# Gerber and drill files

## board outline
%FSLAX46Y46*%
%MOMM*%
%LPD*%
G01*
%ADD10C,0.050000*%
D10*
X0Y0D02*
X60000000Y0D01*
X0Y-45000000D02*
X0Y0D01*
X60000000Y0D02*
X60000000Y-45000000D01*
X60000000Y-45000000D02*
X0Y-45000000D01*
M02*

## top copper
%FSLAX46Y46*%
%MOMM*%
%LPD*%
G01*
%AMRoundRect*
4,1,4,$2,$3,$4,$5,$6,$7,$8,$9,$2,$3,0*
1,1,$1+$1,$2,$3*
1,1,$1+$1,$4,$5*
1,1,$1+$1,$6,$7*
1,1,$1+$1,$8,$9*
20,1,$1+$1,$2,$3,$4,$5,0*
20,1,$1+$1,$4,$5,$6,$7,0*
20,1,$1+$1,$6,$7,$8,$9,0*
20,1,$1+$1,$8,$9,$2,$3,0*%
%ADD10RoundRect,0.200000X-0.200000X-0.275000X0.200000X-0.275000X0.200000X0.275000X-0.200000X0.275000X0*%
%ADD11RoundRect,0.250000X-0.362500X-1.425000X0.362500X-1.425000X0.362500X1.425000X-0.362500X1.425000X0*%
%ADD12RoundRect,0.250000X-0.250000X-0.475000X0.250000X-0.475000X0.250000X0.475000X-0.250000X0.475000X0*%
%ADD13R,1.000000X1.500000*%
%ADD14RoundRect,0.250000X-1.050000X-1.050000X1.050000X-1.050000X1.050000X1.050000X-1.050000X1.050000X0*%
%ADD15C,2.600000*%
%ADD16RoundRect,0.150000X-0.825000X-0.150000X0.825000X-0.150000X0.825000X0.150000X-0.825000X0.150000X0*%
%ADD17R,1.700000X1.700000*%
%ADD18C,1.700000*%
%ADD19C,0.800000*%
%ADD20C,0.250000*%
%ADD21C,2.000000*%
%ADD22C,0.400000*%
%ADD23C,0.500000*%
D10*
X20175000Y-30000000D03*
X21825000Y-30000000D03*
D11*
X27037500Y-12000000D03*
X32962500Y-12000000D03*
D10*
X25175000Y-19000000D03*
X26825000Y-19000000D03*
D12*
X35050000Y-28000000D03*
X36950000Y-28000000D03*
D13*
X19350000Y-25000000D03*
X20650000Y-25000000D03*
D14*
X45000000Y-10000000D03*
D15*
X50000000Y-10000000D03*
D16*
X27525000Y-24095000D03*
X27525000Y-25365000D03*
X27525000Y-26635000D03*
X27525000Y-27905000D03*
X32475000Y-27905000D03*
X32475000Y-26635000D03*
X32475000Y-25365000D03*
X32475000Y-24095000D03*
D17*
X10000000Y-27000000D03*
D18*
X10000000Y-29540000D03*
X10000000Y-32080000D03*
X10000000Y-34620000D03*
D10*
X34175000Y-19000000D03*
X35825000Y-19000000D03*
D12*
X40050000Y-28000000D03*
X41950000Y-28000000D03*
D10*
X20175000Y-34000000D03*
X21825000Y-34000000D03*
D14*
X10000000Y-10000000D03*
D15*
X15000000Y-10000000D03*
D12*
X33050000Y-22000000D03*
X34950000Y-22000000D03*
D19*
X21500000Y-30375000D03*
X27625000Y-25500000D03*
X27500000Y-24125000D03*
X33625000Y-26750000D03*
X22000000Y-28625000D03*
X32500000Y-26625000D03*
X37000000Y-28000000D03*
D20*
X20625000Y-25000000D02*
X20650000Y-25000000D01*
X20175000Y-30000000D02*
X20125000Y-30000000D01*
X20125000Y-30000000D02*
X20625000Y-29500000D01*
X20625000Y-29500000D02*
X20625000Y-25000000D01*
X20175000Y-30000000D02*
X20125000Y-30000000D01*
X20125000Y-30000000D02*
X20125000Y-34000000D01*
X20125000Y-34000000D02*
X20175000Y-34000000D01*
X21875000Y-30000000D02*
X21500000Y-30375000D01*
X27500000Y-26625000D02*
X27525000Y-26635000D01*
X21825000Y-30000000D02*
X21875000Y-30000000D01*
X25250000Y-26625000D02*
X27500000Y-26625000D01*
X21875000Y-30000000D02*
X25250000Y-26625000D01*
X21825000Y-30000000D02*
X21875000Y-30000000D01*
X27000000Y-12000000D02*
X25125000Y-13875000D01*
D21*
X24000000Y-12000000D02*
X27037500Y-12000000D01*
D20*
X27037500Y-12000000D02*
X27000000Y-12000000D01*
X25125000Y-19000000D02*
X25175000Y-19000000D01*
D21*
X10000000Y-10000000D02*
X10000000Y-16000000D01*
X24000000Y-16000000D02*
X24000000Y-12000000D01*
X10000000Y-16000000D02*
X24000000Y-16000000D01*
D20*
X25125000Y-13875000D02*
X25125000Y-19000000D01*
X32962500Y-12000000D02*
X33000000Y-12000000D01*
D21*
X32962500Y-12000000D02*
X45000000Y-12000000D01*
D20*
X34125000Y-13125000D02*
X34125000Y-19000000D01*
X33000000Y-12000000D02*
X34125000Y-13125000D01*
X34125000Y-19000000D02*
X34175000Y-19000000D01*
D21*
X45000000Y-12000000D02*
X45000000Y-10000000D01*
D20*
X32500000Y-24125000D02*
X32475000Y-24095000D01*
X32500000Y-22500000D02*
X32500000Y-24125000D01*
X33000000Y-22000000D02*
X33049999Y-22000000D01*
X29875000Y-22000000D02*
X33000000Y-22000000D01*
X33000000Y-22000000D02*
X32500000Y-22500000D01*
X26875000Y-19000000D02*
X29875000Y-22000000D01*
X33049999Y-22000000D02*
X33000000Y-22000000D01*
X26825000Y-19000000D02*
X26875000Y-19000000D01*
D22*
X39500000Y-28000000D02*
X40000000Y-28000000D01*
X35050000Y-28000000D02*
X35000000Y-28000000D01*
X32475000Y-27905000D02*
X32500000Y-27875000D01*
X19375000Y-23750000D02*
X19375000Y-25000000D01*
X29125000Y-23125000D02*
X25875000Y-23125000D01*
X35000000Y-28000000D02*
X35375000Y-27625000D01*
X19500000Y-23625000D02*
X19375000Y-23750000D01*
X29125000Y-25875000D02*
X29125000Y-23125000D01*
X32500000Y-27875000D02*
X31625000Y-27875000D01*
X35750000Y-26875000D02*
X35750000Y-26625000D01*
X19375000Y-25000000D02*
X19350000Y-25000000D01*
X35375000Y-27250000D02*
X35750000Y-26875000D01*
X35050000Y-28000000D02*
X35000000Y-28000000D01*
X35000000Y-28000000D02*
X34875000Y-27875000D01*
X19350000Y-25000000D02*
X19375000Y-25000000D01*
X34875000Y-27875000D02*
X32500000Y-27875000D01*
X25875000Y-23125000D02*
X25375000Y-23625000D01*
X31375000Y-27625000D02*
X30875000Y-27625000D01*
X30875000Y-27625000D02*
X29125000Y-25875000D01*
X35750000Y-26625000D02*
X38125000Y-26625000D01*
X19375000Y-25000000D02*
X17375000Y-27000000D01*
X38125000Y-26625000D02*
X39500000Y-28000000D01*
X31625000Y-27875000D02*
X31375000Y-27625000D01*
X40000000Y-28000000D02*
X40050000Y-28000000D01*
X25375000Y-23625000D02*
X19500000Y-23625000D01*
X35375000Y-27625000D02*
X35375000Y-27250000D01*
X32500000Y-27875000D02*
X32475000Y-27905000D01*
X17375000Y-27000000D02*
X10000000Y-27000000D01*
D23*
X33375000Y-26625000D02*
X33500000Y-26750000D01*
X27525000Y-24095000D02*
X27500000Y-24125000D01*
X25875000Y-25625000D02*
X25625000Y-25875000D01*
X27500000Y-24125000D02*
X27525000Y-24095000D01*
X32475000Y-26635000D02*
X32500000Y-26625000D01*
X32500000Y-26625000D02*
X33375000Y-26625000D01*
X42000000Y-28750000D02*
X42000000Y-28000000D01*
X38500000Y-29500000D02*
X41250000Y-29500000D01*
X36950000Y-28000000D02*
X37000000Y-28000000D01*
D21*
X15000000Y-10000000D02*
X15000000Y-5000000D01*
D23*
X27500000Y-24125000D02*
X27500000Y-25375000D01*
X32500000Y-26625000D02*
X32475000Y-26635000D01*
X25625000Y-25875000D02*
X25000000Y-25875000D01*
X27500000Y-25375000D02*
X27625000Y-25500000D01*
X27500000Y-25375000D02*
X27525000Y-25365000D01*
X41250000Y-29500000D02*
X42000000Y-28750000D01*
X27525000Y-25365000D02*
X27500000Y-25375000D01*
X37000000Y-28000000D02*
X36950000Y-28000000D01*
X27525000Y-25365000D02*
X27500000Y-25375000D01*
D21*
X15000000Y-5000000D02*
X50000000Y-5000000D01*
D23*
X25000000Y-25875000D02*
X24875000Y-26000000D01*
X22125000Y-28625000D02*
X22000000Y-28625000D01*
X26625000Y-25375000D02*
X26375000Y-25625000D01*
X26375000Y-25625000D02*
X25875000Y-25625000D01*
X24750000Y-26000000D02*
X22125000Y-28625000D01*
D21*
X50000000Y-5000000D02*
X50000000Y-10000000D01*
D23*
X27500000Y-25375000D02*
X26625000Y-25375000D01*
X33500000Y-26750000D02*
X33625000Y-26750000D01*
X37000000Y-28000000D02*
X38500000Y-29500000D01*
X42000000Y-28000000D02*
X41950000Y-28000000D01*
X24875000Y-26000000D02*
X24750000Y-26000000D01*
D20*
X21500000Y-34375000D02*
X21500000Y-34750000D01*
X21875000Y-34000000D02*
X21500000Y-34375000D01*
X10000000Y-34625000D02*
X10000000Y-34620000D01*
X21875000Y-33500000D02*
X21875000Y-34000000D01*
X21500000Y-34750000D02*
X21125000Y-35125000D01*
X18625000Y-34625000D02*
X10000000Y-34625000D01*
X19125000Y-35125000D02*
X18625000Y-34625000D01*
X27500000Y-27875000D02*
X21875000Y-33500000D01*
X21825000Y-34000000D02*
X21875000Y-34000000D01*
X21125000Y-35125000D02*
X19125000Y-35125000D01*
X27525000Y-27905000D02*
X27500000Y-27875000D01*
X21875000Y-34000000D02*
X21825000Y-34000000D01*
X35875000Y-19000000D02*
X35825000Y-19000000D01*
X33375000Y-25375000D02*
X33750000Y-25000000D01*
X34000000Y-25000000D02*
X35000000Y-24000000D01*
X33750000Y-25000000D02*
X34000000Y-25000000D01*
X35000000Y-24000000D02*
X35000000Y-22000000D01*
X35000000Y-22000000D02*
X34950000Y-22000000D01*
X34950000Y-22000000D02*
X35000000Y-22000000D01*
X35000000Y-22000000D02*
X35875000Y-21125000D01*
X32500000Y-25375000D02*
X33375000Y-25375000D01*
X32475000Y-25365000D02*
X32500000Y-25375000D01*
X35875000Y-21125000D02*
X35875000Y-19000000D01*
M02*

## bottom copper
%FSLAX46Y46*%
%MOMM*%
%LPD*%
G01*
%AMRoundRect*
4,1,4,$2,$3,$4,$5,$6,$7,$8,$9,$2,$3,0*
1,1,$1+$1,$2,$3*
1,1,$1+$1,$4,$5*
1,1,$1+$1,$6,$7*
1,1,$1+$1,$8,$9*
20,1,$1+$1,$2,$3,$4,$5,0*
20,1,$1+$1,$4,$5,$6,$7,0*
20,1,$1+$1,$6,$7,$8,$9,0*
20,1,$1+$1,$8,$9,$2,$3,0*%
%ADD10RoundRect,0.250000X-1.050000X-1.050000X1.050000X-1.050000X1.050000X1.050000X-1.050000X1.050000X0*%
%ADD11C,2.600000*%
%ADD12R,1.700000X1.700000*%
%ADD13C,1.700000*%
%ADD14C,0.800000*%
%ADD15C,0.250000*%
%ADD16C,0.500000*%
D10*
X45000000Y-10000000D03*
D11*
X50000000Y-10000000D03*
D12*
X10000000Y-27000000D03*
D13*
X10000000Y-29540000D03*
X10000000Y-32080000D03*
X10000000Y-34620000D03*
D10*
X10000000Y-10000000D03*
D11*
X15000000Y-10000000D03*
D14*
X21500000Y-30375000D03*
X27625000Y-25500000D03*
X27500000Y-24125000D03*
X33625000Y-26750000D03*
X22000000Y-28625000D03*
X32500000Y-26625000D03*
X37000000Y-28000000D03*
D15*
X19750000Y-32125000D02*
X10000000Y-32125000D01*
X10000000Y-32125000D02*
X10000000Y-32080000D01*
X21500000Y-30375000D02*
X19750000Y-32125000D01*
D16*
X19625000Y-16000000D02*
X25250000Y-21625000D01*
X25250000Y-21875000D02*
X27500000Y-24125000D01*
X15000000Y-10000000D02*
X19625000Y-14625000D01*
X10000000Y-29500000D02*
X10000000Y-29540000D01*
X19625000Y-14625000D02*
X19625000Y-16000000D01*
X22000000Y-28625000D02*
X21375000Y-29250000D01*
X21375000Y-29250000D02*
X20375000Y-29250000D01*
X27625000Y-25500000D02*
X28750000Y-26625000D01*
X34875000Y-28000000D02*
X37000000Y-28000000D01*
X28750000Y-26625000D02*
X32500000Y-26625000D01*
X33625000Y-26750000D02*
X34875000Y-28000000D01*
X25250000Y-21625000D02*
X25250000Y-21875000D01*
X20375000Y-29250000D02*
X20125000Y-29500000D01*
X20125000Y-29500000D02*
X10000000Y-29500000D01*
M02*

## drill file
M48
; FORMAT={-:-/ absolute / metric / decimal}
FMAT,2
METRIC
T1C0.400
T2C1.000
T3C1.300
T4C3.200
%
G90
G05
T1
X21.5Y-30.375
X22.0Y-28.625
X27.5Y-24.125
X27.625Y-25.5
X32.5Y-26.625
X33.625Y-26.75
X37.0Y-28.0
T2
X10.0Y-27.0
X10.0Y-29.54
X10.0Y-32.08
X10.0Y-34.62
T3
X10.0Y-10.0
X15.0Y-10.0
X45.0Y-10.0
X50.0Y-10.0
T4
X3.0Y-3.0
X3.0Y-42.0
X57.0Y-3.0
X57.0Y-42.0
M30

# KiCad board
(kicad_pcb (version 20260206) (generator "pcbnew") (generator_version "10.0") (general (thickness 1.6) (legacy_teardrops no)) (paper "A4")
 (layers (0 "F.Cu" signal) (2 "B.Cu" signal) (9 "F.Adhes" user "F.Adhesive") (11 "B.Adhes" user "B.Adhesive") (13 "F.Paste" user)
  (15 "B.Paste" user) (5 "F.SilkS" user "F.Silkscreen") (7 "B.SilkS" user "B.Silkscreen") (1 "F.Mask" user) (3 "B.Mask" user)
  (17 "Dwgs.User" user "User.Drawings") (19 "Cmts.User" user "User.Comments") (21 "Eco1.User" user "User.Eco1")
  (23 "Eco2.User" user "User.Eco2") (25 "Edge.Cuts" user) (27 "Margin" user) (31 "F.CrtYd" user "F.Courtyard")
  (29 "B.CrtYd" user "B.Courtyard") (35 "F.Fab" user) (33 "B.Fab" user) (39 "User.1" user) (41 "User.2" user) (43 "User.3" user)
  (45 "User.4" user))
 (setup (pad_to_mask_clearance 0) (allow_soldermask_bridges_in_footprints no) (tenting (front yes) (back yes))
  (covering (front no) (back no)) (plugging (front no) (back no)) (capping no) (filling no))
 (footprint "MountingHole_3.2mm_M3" (layer "F.Cu") (at 57 3)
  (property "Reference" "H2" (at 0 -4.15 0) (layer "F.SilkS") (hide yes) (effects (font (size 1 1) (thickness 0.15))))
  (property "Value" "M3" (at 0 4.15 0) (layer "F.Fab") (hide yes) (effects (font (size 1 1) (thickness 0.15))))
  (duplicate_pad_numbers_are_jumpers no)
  (pad "" np_thru_hole circle (at 0 0) (size 3.2 3.2) (drill 3.2) (layers "*.Cu" "*.Mask")))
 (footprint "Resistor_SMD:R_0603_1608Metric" (layer "F.Cu") (at 21 30)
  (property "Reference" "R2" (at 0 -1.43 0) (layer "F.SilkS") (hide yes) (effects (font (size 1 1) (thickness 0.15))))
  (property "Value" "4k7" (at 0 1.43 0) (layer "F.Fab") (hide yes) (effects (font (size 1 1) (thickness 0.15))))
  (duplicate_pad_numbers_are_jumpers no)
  (pad "1" smd roundrect (at -0.825 0) (size 0.8 0.95) (layers "F.Cu" "F.Mask" "F.Paste") (roundrect_rratio 0.25) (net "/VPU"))
  (pad "2" smd roundrect (at 0.825 0) (size 0.8 0.95) (layers "F.Cu" "F.Mask" "F.Paste") (roundrect_rratio 0.25) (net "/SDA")))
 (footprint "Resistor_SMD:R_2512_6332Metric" (layer "F.Cu") (at 30 12)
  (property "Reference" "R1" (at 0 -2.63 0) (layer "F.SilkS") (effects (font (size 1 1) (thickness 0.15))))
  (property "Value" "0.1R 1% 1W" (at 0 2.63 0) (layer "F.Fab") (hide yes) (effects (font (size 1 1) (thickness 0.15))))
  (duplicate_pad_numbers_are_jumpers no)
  (pad "1" smd roundrect (at -2.9625 0) (size 1.225 3.35) (layers "F.Cu" "F.Mask" "F.Paste") (roundrect_rratio 0.204082) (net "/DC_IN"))
  (pad "2" smd roundrect (at 2.9625 0) (size 1.225 3.35) (layers "F.Cu" "F.Mask" "F.Paste") (roundrect_rratio 0.204082) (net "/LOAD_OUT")))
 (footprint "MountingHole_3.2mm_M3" (layer "F.Cu") (at 57 42)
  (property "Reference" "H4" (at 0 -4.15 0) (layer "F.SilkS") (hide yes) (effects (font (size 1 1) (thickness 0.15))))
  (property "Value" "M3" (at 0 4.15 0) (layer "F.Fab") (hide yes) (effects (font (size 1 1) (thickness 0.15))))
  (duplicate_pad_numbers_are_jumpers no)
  (pad "" np_thru_hole circle (at 0 0) (size 3.2 3.2) (drill 3.2) (layers "*.Cu" "*.Mask")))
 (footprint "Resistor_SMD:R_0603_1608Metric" (layer "F.Cu") (at 26 19)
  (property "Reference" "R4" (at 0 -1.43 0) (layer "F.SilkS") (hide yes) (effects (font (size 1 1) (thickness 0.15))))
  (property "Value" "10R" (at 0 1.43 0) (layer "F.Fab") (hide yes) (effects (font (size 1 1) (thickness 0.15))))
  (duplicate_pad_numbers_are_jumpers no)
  (pad "1" smd roundrect (at -0.825 0) (size 0.8 0.95) (layers "F.Cu" "F.Mask" "F.Paste") (roundrect_rratio 0.25) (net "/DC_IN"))
  (pad "2" smd roundrect (at 0.825 0) (size 0.8 0.95) (layers "F.Cu" "F.Mask" "F.Paste") (roundrect_rratio 0.25) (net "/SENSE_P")))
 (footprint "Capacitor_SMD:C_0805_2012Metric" (layer "F.Cu") (at 36 28)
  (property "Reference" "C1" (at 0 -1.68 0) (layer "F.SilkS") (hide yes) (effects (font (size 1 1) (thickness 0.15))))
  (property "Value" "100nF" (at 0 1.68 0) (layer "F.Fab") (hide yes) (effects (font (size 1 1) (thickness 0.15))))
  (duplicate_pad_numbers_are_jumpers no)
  (pad "1" smd roundrect (at -0.95 0) (size 1 1.45) (layers "F.Cu" "F.Mask" "F.Paste") (roundrect_rratio 0.25) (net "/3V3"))
  (pad "2" smd roundrect (at 0.95 0) (size 1 1.45) (layers "F.Cu" "F.Mask" "F.Paste") (roundrect_rratio 0.25) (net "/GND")))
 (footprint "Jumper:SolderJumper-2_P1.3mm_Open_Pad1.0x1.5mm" (layer "F.Cu") (at 20 25)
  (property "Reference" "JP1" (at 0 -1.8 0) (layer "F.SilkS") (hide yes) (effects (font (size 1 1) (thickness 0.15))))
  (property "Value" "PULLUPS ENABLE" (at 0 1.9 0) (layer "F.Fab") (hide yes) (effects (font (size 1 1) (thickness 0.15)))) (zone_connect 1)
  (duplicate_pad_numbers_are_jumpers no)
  (pad "1" smd rect (at -0.65 0) (size 1 1.5) (layers "F.Cu" "F.Mask") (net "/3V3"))
  (pad "2" smd rect (at 0.65 0) (size 1 1.5) (layers "F.Cu" "F.Mask") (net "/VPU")))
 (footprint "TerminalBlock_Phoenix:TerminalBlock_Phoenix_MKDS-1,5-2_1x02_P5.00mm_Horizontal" (layer "F.Cu") (at 45 10)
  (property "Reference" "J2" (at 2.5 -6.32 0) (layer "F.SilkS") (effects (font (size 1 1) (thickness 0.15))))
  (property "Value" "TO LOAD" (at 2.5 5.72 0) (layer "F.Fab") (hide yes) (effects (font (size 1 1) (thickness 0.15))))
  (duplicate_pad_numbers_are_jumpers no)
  (pad "1" thru_hole roundrect (at 0 0) (size 2.6 2.6) (drill 1.3) (layers "*.Cu" "*.Mask") (remove_unused_layers no)
   (roundrect_rratio 0.096154) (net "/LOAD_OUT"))
  (pad "2" thru_hole circle (at 5 0) (size 2.6 2.6) (drill 1.3) (layers "*.Cu" "*.Mask") (remove_unused_layers no) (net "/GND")))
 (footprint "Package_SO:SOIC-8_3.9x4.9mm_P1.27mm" (layer "F.Cu") (at 30 26)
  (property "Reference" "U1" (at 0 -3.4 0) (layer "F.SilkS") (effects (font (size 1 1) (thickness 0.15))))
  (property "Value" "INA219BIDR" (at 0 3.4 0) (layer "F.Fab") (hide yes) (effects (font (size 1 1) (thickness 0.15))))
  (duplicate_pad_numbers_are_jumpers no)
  (pad "1" smd roundrect (at -2.475 -1.905) (size 1.95 0.6) (layers "F.Cu" "F.Mask" "F.Paste") (roundrect_rratio 0.25) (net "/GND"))
  (pad "2" smd roundrect (at -2.475 -0.635) (size 1.95 0.6) (layers "F.Cu" "F.Mask" "F.Paste") (roundrect_rratio 0.25) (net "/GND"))
  (pad "3" smd roundrect (at -2.475 0.635) (size 1.95 0.6) (layers "F.Cu" "F.Mask" "F.Paste") (roundrect_rratio 0.25) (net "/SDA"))
  (pad "4" smd roundrect (at -2.475 1.905) (size 1.95 0.6) (layers "F.Cu" "F.Mask" "F.Paste") (roundrect_rratio 0.25) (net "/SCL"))
  (pad "5" smd roundrect (at 2.475 1.905) (size 1.95 0.6) (layers "F.Cu" "F.Mask" "F.Paste") (roundrect_rratio 0.25) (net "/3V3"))
  (pad "6" smd roundrect (at 2.475 0.635) (size 1.95 0.6) (layers "F.Cu" "F.Mask" "F.Paste") (roundrect_rratio 0.25) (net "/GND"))
  (pad "7" smd roundrect (at 2.475 -0.635) (size 1.95 0.6) (layers "F.Cu" "F.Mask" "F.Paste") (roundrect_rratio 0.25) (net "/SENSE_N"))
  (pad "8" smd roundrect (at 2.475 -1.905) (size 1.95 0.6) (layers "F.Cu" "F.Mask" "F.Paste") (roundrect_rratio 0.25) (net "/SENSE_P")))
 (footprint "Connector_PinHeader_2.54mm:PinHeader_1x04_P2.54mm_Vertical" (layer "F.Cu") (at 10 27)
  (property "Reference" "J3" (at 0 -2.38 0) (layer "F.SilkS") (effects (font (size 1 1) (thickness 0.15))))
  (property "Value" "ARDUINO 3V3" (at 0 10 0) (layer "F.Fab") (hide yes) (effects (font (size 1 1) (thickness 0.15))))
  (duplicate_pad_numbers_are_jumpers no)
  (pad "1" thru_hole rect (at 0 0) (size 1.7 1.7) (drill 1) (layers "*.Cu" "*.Mask") (remove_unused_layers no) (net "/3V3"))
  (pad "2" thru_hole circle (at 0 2.54) (size 1.7 1.7) (drill 1) (layers "*.Cu" "*.Mask") (remove_unused_layers no) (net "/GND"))
  (pad "3" thru_hole circle (at 0 5.08) (size 1.7 1.7) (drill 1) (layers "*.Cu" "*.Mask") (remove_unused_layers no) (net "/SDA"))
  (pad "4" thru_hole circle (at 0 7.62) (size 1.7 1.7) (drill 1) (layers "*.Cu" "*.Mask") (remove_unused_layers no) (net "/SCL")))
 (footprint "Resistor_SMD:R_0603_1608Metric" (layer "F.Cu") (at 35 19)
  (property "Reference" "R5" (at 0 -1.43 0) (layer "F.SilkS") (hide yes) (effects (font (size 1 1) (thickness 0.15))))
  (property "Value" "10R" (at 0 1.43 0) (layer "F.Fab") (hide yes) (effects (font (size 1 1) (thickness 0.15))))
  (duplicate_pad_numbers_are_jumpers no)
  (pad "1" smd roundrect (at -0.825 0) (size 0.8 0.95) (layers "F.Cu" "F.Mask" "F.Paste") (roundrect_rratio 0.25) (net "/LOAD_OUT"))
  (pad "2" smd roundrect (at 0.825 0) (size 0.8 0.95) (layers "F.Cu" "F.Mask" "F.Paste") (roundrect_rratio 0.25) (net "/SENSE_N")))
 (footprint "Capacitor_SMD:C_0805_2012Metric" (layer "F.Cu") (at 41 28)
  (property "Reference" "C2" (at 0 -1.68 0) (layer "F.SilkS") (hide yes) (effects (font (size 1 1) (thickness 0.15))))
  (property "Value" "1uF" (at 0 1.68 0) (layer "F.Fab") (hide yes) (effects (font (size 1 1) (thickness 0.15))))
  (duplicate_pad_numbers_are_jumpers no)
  (pad "1" smd roundrect (at -0.95 0) (size 1 1.45) (layers "F.Cu" "F.Mask" "F.Paste") (roundrect_rratio 0.25) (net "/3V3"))
  (pad "2" smd roundrect (at 0.95 0) (size 1 1.45) (layers "F.Cu" "F.Mask" "F.Paste") (roundrect_rratio 0.25) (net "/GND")))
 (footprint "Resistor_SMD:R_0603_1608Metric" (layer "F.Cu") (at 21 34)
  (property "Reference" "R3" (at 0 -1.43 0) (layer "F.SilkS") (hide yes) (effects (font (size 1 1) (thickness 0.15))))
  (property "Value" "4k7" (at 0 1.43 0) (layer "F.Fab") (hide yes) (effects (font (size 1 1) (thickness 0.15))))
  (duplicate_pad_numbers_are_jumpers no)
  (pad "1" smd roundrect (at -0.825 0) (size 0.8 0.95) (layers "F.Cu" "F.Mask" "F.Paste") (roundrect_rratio 0.25) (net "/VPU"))
  (pad "2" smd roundrect (at 0.825 0) (size 0.8 0.95) (layers "F.Cu" "F.Mask" "F.Paste") (roundrect_rratio 0.25) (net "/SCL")))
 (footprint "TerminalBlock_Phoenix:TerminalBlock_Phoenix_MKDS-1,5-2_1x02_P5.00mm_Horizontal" (layer "F.Cu") (at 10 10)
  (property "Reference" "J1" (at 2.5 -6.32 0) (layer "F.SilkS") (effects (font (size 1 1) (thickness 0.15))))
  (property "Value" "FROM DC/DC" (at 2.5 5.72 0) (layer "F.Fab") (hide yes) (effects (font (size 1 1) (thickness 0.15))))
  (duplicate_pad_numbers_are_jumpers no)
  (pad "1" thru_hole roundrect (at 0 0) (size 2.6 2.6) (drill 1.3) (layers "*.Cu" "*.Mask") (remove_unused_layers no)
   (roundrect_rratio 0.096154) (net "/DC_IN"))
  (pad "2" thru_hole circle (at 5 0) (size 2.6 2.6) (drill 1.3) (layers "*.Cu" "*.Mask") (remove_unused_layers no) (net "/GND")))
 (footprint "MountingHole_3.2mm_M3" (layer "F.Cu") (at 3 3)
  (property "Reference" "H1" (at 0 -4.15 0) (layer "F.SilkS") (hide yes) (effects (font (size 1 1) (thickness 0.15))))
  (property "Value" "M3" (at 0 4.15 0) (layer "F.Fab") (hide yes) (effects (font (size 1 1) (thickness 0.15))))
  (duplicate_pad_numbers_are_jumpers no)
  (pad "" np_thru_hole circle (at 0 0) (size 3.2 3.2) (drill 3.2) (layers "*.Cu" "*.Mask")))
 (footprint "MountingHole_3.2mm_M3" (layer "F.Cu") (at 3 42)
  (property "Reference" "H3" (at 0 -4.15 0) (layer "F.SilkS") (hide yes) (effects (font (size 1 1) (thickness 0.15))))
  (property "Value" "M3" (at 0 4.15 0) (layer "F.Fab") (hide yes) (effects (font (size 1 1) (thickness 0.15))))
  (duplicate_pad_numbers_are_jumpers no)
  (pad "" np_thru_hole circle (at 0 0) (size 3.2 3.2) (drill 3.2) (layers "*.Cu" "*.Mask")))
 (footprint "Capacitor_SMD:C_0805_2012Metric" (layer "F.Cu") (at 34 22)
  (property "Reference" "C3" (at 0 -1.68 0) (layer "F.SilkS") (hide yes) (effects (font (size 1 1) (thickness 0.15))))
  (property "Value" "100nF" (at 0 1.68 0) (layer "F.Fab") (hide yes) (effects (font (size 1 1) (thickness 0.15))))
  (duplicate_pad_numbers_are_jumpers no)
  (pad "1" smd roundrect (at -0.95 0) (size 1 1.45) (layers "F.Cu" "F.Mask" "F.Paste") (roundrect_rratio 0.25) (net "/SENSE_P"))
  (pad "2" smd roundrect (at 0.95 0) (size 1 1.45) (layers "F.Cu" "F.Mask" "F.Paste") (roundrect_rratio 0.25) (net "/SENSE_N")))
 (gr_line (start 0 0) (end 60 0) (stroke (width 0.05) (type default)) (layer "Edge.Cuts"))
 (gr_line (start 0 45) (end 0 0) (stroke (width 0.05) (type default)) (layer "Edge.Cuts"))
 (gr_line (start 60 0) (end 60 45) (stroke (width 0.05) (type default)) (layer "Edge.Cuts"))
 (gr_line (start 60 45) (end 0 45) (stroke (width 0.05) (type default)) (layer "Edge.Cuts"))
 (segment (start 20.625 25) (end 20.65 25) (width 0.25) (layer "F.Cu") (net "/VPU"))
 (segment (start 20.175 30) (end 20.125 30) (width 0.25) (layer "F.Cu") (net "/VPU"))
 (segment (start 20.125 30) (end 20.625 29.5) (width 0.25) (layer "F.Cu") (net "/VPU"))
 (segment (start 20.625 29.5) (end 20.625 25) (width 0.25) (layer "F.Cu") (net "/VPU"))
 (segment (start 20.175 30) (end 20.125 30) (width 0.25) (layer "F.Cu") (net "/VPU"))
 (segment (start 20.125 30) (end 20.125 34) (width 0.25) (layer "F.Cu") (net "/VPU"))
 (segment (start 20.125 34) (end 20.175 34) (width 0.25) (layer "F.Cu") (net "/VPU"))
 (segment (start 21.875 30) (end 21.5 30.375) (width 0.25) (layer "F.Cu") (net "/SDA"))
 (segment (start 27.5 26.625) (end 27.525 26.635) (width 0.25) (layer "F.Cu") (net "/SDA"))
 (segment (start 21.825 30) (end 21.875 30) (width 0.25) (layer "F.Cu") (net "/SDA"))
 (segment (start 25.25 26.625) (end 27.5 26.625) (width 0.25) (layer "F.Cu") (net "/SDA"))
 (segment (start 21.875 30) (end 25.25 26.625) (width 0.25) (layer "F.Cu") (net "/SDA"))
 (segment (start 21.825 30) (end 21.875 30) (width 0.25) (layer "F.Cu") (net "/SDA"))
 (via (at 21.5 30.375) (size 0.8) (drill 0.4) (layers "F.Cu" "B.Cu") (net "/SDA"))
 (segment (start 19.75 32.125) (end 10 32.125) (width 0.25) (layer "B.Cu") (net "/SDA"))
 (segment (start 10 32.125) (end 10 32.08) (width 0.25) (layer "B.Cu") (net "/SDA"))
 (segment (start 21.5 30.375) (end 19.75 32.125) (width 0.25) (layer "B.Cu") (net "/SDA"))
 (segment (start 27 12) (end 25.125 13.875) (width 0.25) (layer "F.Cu") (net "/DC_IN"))
 (segment (start 24 12) (end 27.0375 12) (width 2) (layer "F.Cu") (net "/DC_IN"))
 (segment (start 27.0375 12) (end 27 12) (width 0.25) (layer "F.Cu") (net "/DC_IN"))
 (segment (start 25.125 19) (end 25.175 19) (width 0.25) (layer "F.Cu") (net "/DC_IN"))
 (segment (start 10 10) (end 10 16) (width 2) (layer "F.Cu") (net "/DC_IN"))
 (segment (start 24 16) (end 24 12) (width 2) (layer "F.Cu") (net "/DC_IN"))
 (segment (start 10 16) (end 24 16) (width 2) (layer "F.Cu") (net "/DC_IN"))
 (segment (start 25.125 13.875) (end 25.125 19) (width 0.25) (layer "F.Cu") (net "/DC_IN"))
 (segment (start 32.9625 12) (end 33 12) (width 0.25) (layer "F.Cu") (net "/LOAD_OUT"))
 (segment (start 32.9625 12) (end 45 12) (width 2) (layer "F.Cu") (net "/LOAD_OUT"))
 (segment (start 34.125 13.125) (end 34.125 19) (width 0.25) (layer "F.Cu") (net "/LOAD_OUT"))
 (segment (start 33 12) (end 34.125 13.125) (width 0.25) (layer "F.Cu") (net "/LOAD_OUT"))
 (segment (start 34.125 19) (end 34.175 19) (width 0.25) (layer "F.Cu") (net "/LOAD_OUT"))
 (segment (start 45 12) (end 45 10) (width 2) (layer "F.Cu") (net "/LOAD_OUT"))
 (segment (start 32.5 24.125) (end 32.475 24.095) (width 0.25) (layer "F.Cu") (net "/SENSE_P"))
 (segment (start 32.5 22.5) (end 32.5 24.125) (width 0.25) (layer "F.Cu") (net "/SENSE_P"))
 (segment (start 33 22) (end 33.049999 22) (width 0.25) (layer "F.Cu") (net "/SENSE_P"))
 (segment (start 29.875 22) (end 33 22) (width 0.25) (layer "F.Cu") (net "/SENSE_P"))
 (segment (start 33 22) (end 32.5 22.5) (width 0.25) (layer "F.Cu") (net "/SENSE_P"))
 (segment (start 26.875 19) (end 29.875 22) (width 0.25) (layer "F.Cu") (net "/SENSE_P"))
 (segment (start 33.049999 22) (end 33 22) (width 0.25) (layer "F.Cu") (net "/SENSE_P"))
 (segment (start 26.825 19) (end 26.875 19) (width 0.25) (layer "F.Cu") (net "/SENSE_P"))
 (segment (start 39.5 28) (end 40 28) (width 0.4) (layer "F.Cu") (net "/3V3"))
 (segment (start 35.05 28) (end 35 28) (width 0.4) (layer "F.Cu") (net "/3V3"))
 (segment (start 32.475 27.905) (end 32.5 27.875) (width 0.4) (layer "F.Cu") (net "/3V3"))
 (segment (start 19.375 23.75) (end 19.375 25) (width 0.4) (layer "F.Cu") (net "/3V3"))
 (segment (start 29.125 23.125) (end 25.875 23.125) (width 0.4) (layer "F.Cu") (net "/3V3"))
 (segment (start 35 28) (end 35.375 27.625) (width 0.4) (layer "F.Cu") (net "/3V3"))
 (segment (start 19.5 23.625) (end 19.375 23.75) (width 0.4) (layer "F.Cu") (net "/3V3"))
 (segment (start 29.125 25.875) (end 29.125 23.125) (width 0.4) (layer "F.Cu") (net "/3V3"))
 (segment (start 32.5 27.875) (end 31.625 27.875) (width 0.4) (layer "F.Cu") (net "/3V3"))
 (segment (start 35.75 26.875) (end 35.75 26.625) (width 0.4) (layer "F.Cu") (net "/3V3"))
 (segment (start 19.375 25) (end 19.35 25) (width 0.4) (layer "F.Cu") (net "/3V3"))
 (segment (start 35.375 27.25) (end 35.75 26.875) (width 0.4) (layer "F.Cu") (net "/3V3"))
 (segment (start 35.05 28) (end 35 28) (width 0.4) (layer "F.Cu") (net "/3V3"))
 (segment (start 35 28) (end 34.875 27.875) (width 0.4) (layer "F.Cu") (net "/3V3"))
 (segment (start 19.35 25) (end 19.375 25) (width 0.4) (layer "F.Cu") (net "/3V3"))
 (segment (start 34.875 27.875) (end 32.5 27.875) (width 0.4) (layer "F.Cu") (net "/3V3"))
 (segment (start 25.875 23.125) (end 25.375 23.625) (width 0.4) (layer "F.Cu") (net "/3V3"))
 (segment (start 31.375 27.625) (end 30.875 27.625) (width 0.4) (layer "F.Cu") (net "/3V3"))
 (segment (start 30.875 27.625) (end 29.125 25.875) (width 0.4) (layer "F.Cu") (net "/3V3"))
 (segment (start 35.75 26.625) (end 38.125 26.625) (width 0.4) (layer "F.Cu") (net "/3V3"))
 (segment (start 19.375 25) (end 17.375 27) (width 0.4) (layer "F.Cu") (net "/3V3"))
 (segment (start 38.125 26.625) (end 39.5 28) (width 0.4) (layer "F.Cu") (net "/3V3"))
 (segment (start 31.625 27.875) (end 31.375 27.625) (width 0.4) (layer "F.Cu") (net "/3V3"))
 (segment (start 40 28) (end 40.05 28) (width 0.4) (layer "F.Cu") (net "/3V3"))
 (segment (start 25.375 23.625) (end 19.5 23.625) (width 0.4) (layer "F.Cu") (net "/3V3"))
 (segment (start 35.375 27.625) (end 35.375 27.25) (width 0.4) (layer "F.Cu") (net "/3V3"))
 (segment (start 32.5 27.875) (end 32.475 27.905) (width 0.4) (layer "F.Cu") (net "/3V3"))
 (segment (start 17.375 27) (end 10 27) (width 0.4) (layer "F.Cu") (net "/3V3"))
 (segment (start 33.375 26.625) (end 33.5 26.75) (width 0.5) (layer "F.Cu") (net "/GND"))
 (segment (start 27.525 24.095) (end 27.5 24.125) (width 0.5) (layer "F.Cu") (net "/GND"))
 (segment (start 25.875 25.625) (end 25.625 25.875) (width 0.5) (layer "F.Cu") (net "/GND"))
 (segment (start 27.5 24.125) (end 27.525 24.095) (width 0.5) (layer "F.Cu") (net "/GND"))
 (segment (start 32.475 26.635) (end 32.5 26.625) (width 0.5) (layer "F.Cu") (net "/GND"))
 (segment (start 32.5 26.625) (end 33.375 26.625) (width 0.5) (layer "F.Cu") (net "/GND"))
 (segment (start 42 28.75) (end 42 28) (width 0.5) (layer "F.Cu") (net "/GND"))
 (segment (start 38.5 29.5) (end 41.25 29.5) (width 0.5) (layer "F.Cu") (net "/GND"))
 (segment (start 36.95 28) (end 37 28) (width 0.5) (layer "F.Cu") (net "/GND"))
 (segment (start 15 10) (end 15 5) (width 2) (layer "F.Cu") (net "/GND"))
 (segment (start 27.5 24.125) (end 27.5 25.375) (width 0.5) (layer "F.Cu") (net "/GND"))
 (segment (start 32.5 26.625) (end 32.475 26.635) (width 0.5) (layer "F.Cu") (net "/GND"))
 (segment (start 25.625 25.875) (end 25 25.875) (width 0.5) (layer "F.Cu") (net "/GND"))
 (segment (start 27.5 25.375) (end 27.625 25.5) (width 0.5) (layer "F.Cu") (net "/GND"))
 (segment (start 27.5 25.375) (end 27.525 25.365) (width 0.5) (layer "F.Cu") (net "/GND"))
 (segment (start 41.25 29.5) (end 42 28.75) (width 0.5) (layer "F.Cu") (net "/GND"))
 (segment (start 27.525 25.365) (end 27.5 25.375) (width 0.5) (layer "F.Cu") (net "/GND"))
 (segment (start 37 28) (end 36.95 28) (width 0.5) (layer "F.Cu") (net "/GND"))
 (segment (start 27.525 25.365) (end 27.5 25.375) (width 0.5) (layer "F.Cu") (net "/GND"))
 (segment (start 15 5) (end 50 5) (width 2) (layer "F.Cu") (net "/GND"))
 (segment (start 25 25.875) (end 24.875 26) (width 0.5) (layer "F.Cu") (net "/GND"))
 (segment (start 22.125 28.625) (end 22 28.625) (width 0.5) (layer "F.Cu") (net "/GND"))
 (segment (start 26.625 25.375) (end 26.375 25.625) (width 0.5) (layer "F.Cu") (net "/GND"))
 (segment (start 26.375 25.625) (end 25.875 25.625) (width 0.5) (layer "F.Cu") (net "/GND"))
 (segment (start 24.75 26) (end 22.125 28.625) (width 0.5) (layer "F.Cu") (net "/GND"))
 (segment (start 50 5) (end 50 10) (width 2) (layer "F.Cu") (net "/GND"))
 (segment (start 27.5 25.375) (end 26.625 25.375) (width 0.5) (layer "F.Cu") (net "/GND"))
 (segment (start 33.5 26.75) (end 33.625 26.75) (width 0.5) (layer "F.Cu") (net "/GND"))
 (segment (start 37 28) (end 38.5 29.5) (width 0.5) (layer "F.Cu") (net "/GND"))
 (segment (start 42 28) (end 41.95 28) (width 0.5) (layer "F.Cu") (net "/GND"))
 (segment (start 24.875 26) (end 24.75 26) (width 0.5) (layer "F.Cu") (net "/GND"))
 (via (at 27.625 25.5) (size 0.8) (drill 0.4) (layers "F.Cu" "B.Cu") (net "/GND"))
 (via (at 27.5 24.125) (size 0.8) (drill 0.4) (layers "F.Cu" "B.Cu") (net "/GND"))
 (via (at 33.625 26.75) (size 0.8) (drill 0.4) (layers "F.Cu" "B.Cu") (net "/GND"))
 (via (at 22 28.625) (size 0.8) (drill 0.4) (layers "F.Cu" "B.Cu") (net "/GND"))
 (via (at 32.5 26.625) (size 0.8) (drill 0.4) (layers "F.Cu" "B.Cu") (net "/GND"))
 (via (at 37 28) (size 0.8) (drill 0.4) (layers "F.Cu" "B.Cu") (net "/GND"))
 (segment (start 19.625 16) (end 25.25 21.625) (width 0.5) (layer "B.Cu") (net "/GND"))
 (segment (start 25.25 21.875) (end 27.5 24.125) (width 0.5) (layer "B.Cu") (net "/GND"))
 (segment (start 15 10) (end 19.625 14.625) (width 0.5) (layer "B.Cu") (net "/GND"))
 (segment (start 10 29.5) (end 10 29.54) (width 0.5) (layer "B.Cu") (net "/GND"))
 (segment (start 19.625 14.625) (end 19.625 16) (width 0.5) (layer "B.Cu") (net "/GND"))
 (segment (start 22 28.625) (end 21.375 29.25) (width 0.5) (layer "B.Cu") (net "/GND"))
 (segment (start 21.375 29.25) (end 20.375 29.25) (width 0.5) (layer "B.Cu") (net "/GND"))
 (segment (start 27.625 25.5) (end 28.75 26.625) (width 0.5) (layer "B.Cu") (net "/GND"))
 (segment (start 34.875 28) (end 37 28) (width 0.5) (layer "B.Cu") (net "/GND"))
 (segment (start 28.75 26.625) (end 32.5 26.625) (width 0.5) (layer "B.Cu") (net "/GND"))
 (segment (start 33.625 26.75) (end 34.875 28) (width 0.5) (layer "B.Cu") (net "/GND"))
 (segment (start 25.25 21.625) (end 25.25 21.875) (width 0.5) (layer "B.Cu") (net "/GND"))
 (segment (start 20.375 29.25) (end 20.125 29.5) (width 0.5) (layer "B.Cu") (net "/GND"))
 (segment (start 20.125 29.5) (end 10 29.5) (width 0.5) (layer "B.Cu") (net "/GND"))
 (segment (start 21.5 34.375) (end 21.5 34.75) (width 0.25) (layer "F.Cu") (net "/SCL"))
 (segment (start 21.875 34) (end 21.5 34.375) (width 0.25) (layer "F.Cu") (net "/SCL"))
 (segment (start 10 34.625) (end 10 34.62) (width 0.25) (layer "F.Cu") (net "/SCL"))
 (segment (start 21.875 33.5) (end 21.875 34) (width 0.25) (layer "F.Cu") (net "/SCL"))
 (segment (start 21.5 34.75) (end 21.125 35.125) (width 0.25) (layer "F.Cu") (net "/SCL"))
 (segment (start 18.625 34.625) (end 10 34.625) (width 0.25) (layer "F.Cu") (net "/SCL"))
 (segment (start 19.125 35.125) (end 18.625 34.625) (width 0.25) (layer "F.Cu") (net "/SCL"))
 (segment (start 27.5 27.875) (end 21.875 33.5) (width 0.25) (layer "F.Cu") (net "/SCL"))
 (segment (start 21.825 34) (end 21.875 34) (width 0.25) (layer "F.Cu") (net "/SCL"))
 (segment (start 21.125 35.125) (end 19.125 35.125) (width 0.25) (layer "F.Cu") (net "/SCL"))
 (segment (start 27.525 27.905) (end 27.5 27.875) (width 0.25) (layer "F.Cu") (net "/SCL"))
 (segment (start 21.875 34) (end 21.825 34) (width 0.25) (layer "F.Cu") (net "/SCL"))
 (segment (start 35.875 19) (end 35.825 19) (width 0.25) (layer "F.Cu") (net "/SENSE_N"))
 (segment (start 33.375 25.375) (end 33.75 25) (width 0.25) (layer "F.Cu") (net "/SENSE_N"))
 (segment (start 34 25) (end 35 24) (width 0.25) (layer "F.Cu") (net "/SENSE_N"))
 (segment (start 33.75 25) (end 34 25) (width 0.25) (layer "F.Cu") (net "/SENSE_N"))
 (segment (start 35 24) (end 35 22) (width 0.25) (layer "F.Cu") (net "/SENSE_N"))
 (segment (start 35 22) (end 34.95 22) (width 0.25) (layer "F.Cu") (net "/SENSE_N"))
 (segment (start 34.95 22) (end 35 22) (width 0.25) (layer "F.Cu") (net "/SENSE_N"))
 (segment (start 35 22) (end 35.875 21.125) (width 0.25) (layer "F.Cu") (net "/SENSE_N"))
 (segment (start 32.5 25.375) (end 33.375 25.375) (width 0.25) (layer "F.Cu") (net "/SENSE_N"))
 (segment (start 32.475 25.365) (end 32.5 25.375) (width 0.25) (layer "F.Cu") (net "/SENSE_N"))
 (segment (start 35.875 21.125) (end 35.875 19) (width 0.25) (layer "F.Cu") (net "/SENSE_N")))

